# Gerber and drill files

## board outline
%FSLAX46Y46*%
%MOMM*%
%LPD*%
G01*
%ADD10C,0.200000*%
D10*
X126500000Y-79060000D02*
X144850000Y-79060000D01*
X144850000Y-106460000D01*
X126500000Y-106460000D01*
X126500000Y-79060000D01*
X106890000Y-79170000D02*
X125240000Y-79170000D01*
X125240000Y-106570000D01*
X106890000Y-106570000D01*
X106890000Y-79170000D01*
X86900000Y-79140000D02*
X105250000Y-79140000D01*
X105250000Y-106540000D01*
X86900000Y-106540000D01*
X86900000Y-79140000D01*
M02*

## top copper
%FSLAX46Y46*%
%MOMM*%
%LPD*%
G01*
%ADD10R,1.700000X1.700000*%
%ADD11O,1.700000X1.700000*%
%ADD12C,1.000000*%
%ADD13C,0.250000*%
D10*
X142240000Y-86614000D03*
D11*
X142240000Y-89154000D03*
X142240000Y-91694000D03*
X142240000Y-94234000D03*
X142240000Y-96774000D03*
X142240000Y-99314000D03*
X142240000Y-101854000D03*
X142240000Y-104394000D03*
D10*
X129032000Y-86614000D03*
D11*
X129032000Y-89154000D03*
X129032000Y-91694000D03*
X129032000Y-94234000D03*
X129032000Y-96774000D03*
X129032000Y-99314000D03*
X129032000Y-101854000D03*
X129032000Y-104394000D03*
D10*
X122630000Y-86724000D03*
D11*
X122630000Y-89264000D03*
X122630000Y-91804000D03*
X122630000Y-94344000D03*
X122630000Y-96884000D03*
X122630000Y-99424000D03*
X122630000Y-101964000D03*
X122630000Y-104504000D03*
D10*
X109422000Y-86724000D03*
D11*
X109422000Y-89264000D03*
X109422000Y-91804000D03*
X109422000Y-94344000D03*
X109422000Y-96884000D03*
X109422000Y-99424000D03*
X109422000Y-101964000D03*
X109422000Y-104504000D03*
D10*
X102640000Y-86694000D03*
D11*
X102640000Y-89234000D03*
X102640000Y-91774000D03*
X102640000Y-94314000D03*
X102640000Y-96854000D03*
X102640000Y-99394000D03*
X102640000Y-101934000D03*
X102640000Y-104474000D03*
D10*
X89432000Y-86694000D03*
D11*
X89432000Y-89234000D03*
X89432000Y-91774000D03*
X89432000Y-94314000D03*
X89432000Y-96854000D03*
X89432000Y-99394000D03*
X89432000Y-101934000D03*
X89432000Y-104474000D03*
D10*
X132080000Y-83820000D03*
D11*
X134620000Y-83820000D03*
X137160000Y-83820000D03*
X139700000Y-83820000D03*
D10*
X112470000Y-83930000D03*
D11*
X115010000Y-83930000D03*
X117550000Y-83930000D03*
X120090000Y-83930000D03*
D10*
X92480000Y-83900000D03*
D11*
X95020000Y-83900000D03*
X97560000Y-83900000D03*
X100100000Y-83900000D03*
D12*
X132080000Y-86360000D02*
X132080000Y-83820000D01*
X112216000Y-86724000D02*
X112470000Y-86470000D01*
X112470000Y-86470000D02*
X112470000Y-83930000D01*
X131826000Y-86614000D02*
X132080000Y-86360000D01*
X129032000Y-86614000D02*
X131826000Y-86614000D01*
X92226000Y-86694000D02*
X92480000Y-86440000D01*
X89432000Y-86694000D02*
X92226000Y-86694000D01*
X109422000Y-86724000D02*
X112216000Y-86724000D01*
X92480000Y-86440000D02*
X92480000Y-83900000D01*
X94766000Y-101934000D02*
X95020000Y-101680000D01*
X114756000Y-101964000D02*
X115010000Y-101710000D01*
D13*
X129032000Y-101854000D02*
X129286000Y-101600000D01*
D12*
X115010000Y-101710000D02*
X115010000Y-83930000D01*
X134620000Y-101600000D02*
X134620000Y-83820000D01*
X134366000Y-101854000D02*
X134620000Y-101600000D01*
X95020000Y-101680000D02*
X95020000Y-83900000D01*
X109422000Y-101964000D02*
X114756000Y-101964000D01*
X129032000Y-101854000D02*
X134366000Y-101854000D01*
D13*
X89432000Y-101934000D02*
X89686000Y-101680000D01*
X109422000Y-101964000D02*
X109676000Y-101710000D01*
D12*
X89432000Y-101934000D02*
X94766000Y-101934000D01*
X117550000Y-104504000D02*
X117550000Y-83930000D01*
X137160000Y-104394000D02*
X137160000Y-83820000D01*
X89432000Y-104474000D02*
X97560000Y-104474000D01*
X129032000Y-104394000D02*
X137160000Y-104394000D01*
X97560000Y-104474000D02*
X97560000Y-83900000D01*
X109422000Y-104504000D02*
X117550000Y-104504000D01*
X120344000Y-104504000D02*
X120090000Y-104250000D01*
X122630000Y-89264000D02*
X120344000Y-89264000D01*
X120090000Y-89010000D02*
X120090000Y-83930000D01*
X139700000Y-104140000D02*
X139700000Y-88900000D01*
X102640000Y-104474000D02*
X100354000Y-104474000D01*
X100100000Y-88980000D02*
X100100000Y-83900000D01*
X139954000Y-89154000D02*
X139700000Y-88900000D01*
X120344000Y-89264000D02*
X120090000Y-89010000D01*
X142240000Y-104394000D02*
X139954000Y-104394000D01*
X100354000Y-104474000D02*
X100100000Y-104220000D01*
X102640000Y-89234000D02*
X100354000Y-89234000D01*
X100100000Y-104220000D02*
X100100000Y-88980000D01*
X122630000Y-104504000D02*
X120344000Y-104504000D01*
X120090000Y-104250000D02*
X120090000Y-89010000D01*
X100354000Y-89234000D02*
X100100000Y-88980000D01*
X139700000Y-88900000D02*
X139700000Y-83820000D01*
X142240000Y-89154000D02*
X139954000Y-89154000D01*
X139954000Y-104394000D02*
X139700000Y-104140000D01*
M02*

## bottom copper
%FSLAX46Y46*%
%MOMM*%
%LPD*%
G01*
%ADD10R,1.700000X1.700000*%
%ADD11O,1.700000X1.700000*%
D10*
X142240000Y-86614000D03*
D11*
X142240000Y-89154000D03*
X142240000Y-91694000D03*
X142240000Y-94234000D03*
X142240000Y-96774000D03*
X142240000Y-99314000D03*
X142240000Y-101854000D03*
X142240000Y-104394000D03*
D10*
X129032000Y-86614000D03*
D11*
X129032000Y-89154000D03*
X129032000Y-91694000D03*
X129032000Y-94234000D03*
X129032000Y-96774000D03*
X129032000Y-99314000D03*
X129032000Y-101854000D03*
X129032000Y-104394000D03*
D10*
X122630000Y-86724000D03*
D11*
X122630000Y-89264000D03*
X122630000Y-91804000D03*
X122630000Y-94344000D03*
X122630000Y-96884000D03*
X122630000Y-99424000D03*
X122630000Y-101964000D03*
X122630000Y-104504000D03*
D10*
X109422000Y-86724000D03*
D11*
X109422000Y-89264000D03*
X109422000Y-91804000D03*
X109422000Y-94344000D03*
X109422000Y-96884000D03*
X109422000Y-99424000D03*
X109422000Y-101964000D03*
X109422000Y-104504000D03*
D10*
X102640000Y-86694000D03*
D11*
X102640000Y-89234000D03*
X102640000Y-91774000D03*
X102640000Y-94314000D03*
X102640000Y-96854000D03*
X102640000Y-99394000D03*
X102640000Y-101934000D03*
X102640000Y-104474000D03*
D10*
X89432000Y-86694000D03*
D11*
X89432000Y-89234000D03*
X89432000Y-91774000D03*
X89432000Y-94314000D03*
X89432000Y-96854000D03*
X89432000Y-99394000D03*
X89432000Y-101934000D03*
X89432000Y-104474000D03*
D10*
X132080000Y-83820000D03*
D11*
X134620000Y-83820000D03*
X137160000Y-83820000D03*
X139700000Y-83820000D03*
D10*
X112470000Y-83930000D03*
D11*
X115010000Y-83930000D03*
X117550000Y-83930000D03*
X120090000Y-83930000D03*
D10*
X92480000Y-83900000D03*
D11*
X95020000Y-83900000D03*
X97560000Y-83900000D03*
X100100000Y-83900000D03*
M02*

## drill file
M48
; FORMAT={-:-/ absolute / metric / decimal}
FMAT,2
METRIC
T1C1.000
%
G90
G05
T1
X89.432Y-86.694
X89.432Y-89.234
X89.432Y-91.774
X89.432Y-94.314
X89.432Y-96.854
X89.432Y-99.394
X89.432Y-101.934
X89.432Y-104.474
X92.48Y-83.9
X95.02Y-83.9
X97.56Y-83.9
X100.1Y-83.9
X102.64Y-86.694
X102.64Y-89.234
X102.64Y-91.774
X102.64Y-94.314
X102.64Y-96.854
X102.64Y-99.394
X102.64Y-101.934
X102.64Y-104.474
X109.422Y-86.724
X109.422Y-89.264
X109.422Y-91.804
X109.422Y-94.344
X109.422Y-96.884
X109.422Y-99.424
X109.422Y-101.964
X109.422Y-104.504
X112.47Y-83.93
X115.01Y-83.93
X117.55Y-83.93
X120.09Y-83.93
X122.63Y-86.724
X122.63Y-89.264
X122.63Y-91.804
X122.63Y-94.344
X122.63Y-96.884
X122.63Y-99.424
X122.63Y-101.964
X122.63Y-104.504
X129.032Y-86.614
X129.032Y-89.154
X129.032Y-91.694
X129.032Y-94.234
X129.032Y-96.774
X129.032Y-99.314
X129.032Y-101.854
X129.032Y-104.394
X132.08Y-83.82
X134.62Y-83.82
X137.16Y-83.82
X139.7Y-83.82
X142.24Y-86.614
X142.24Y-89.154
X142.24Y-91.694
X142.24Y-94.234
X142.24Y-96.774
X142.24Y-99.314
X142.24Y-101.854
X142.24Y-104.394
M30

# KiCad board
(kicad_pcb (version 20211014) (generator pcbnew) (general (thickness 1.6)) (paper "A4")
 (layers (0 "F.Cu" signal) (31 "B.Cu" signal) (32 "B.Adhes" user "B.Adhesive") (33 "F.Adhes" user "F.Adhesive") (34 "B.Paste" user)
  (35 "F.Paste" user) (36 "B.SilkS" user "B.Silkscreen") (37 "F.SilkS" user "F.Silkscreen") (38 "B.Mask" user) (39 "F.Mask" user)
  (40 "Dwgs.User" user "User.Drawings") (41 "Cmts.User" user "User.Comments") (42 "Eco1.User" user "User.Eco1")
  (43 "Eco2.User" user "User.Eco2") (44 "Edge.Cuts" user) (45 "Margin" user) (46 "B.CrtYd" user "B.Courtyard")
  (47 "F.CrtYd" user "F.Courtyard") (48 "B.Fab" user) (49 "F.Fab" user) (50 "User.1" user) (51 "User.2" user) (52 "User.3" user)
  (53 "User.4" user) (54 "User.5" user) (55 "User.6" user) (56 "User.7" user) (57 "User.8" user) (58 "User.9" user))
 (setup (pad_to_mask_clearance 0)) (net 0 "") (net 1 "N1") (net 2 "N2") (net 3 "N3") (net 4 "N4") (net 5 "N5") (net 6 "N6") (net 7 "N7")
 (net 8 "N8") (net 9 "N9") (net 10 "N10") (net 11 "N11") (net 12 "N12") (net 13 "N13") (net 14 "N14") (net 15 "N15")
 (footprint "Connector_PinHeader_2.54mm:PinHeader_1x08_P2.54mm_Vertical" (layer "F.Cu") (at 142.24 86.614)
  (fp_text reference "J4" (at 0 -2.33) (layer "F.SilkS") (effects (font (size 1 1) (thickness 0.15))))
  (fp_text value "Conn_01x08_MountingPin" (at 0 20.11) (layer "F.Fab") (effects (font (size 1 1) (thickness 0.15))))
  (pad "1" thru_hole rect (at 0 0) (size 1.7 1.7) (drill 1) (layers *.Cu *.Mask) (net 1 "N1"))
  (pad "2" thru_hole oval (at 0 2.54) (size 1.7 1.7) (drill 1) (layers *.Cu *.Mask) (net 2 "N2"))
  (pad "3" thru_hole oval (at 0 5.08) (size 1.7 1.7) (drill 1) (layers *.Cu *.Mask) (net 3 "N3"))
  (pad "4" thru_hole oval (at 0 7.62) (size 1.7 1.7) (drill 1) (layers *.Cu *.Mask) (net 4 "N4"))
  (pad "5" thru_hole oval (at 0 10.16) (size 1.7 1.7) (drill 1) (layers *.Cu *.Mask) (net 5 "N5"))
  (pad "6" thru_hole oval (at 0 12.7) (size 1.7 1.7) (drill 1) (layers *.Cu *.Mask) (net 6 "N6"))
  (pad "7" thru_hole oval (at 0 15.24) (size 1.7 1.7) (drill 1) (layers *.Cu *.Mask) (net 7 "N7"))
  (pad "8" thru_hole oval (at 0 17.78) (size 1.7 1.7) (drill 1) (layers *.Cu *.Mask) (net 2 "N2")))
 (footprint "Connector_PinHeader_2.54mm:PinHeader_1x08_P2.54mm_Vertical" (layer "F.Cu") (at 129.032 86.614)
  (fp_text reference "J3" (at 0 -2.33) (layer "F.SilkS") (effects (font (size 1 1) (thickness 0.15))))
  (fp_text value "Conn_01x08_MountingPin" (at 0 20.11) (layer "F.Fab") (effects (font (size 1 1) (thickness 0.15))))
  (pad "1" thru_hole rect (at 0 0) (size 1.7 1.7) (drill 1) (layers *.Cu *.Mask) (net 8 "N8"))
  (pad "2" thru_hole oval (at 0 2.54) (size 1.7 1.7) (drill 1) (layers *.Cu *.Mask) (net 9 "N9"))
  (pad "3" thru_hole oval (at 0 5.08) (size 1.7 1.7) (drill 1) (layers *.Cu *.Mask) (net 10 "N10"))
  (pad "4" thru_hole oval (at 0 7.62) (size 1.7 1.7) (drill 1) (layers *.Cu *.Mask) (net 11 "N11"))
  (pad "5" thru_hole oval (at 0 10.16) (size 1.7 1.7) (drill 1) (layers *.Cu *.Mask) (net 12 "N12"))
  (pad "6" thru_hole oval (at 0 12.7) (size 1.7 1.7) (drill 1) (layers *.Cu *.Mask) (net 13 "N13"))
  (pad "7" thru_hole oval (at 0 15.24) (size 1.7 1.7) (drill 1) (layers *.Cu *.Mask) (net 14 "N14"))
  (pad "8" thru_hole oval (at 0 17.78) (size 1.7 1.7) (drill 1) (layers *.Cu *.Mask) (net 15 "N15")))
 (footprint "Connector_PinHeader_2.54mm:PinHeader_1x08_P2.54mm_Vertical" (layer "F.Cu") (at 122.63 86.724)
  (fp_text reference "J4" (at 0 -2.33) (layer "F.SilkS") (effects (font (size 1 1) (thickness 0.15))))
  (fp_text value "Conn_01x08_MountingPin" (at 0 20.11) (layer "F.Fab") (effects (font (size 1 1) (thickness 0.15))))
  (pad "1" thru_hole rect (at 0 0) (size 1.7 1.7) (drill 1) (layers *.Cu *.Mask) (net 1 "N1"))
  (pad "2" thru_hole oval (at 0 2.54) (size 1.7 1.7) (drill 1) (layers *.Cu *.Mask) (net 2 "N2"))
  (pad "3" thru_hole oval (at 0 5.08) (size 1.7 1.7) (drill 1) (layers *.Cu *.Mask) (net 3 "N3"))
  (pad "4" thru_hole oval (at 0 7.62) (size 1.7 1.7) (drill 1) (layers *.Cu *.Mask) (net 4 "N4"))
  (pad "5" thru_hole oval (at 0 10.16) (size 1.7 1.7) (drill 1) (layers *.Cu *.Mask) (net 5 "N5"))
  (pad "6" thru_hole oval (at 0 12.7) (size 1.7 1.7) (drill 1) (layers *.Cu *.Mask) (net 6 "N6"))
  (pad "7" thru_hole oval (at 0 15.24) (size 1.7 1.7) (drill 1) (layers *.Cu *.Mask) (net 7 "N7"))
  (pad "8" thru_hole oval (at 0 17.78) (size 1.7 1.7) (drill 1) (layers *.Cu *.Mask) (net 2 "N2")))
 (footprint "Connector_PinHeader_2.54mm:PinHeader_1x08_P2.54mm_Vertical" (layer "F.Cu") (at 109.422 86.724)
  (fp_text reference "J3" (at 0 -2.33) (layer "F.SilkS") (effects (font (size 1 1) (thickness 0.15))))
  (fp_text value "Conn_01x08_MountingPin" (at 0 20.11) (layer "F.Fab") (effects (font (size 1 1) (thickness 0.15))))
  (pad "1" thru_hole rect (at 0 0) (size 1.7 1.7) (drill 1) (layers *.Cu *.Mask) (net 8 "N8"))
  (pad "2" thru_hole oval (at 0 2.54) (size 1.7 1.7) (drill 1) (layers *.Cu *.Mask) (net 9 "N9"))
  (pad "3" thru_hole oval (at 0 5.08) (size 1.7 1.7) (drill 1) (layers *.Cu *.Mask) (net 10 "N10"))
  (pad "4" thru_hole oval (at 0 7.62) (size 1.7 1.7) (drill 1) (layers *.Cu *.Mask) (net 11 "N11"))
  (pad "5" thru_hole oval (at 0 10.16) (size 1.7 1.7) (drill 1) (layers *.Cu *.Mask) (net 12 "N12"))
  (pad "6" thru_hole oval (at 0 12.7) (size 1.7 1.7) (drill 1) (layers *.Cu *.Mask) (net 13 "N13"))
  (pad "7" thru_hole oval (at 0 15.24) (size 1.7 1.7) (drill 1) (layers *.Cu *.Mask) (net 14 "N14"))
  (pad "8" thru_hole oval (at 0 17.78) (size 1.7 1.7) (drill 1) (layers *.Cu *.Mask) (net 15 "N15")))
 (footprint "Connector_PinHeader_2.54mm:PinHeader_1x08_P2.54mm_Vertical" (layer "F.Cu") (at 102.64 86.694)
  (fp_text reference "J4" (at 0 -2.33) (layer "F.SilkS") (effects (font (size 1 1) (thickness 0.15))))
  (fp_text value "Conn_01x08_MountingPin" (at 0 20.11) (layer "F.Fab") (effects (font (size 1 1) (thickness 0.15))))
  (pad "1" thru_hole rect (at 0 0) (size 1.7 1.7) (drill 1) (layers *.Cu *.Mask) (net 1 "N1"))
  (pad "2" thru_hole oval (at 0 2.54) (size 1.7 1.7) (drill 1) (layers *.Cu *.Mask) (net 2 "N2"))
  (pad "3" thru_hole oval (at 0 5.08) (size 1.7 1.7) (drill 1) (layers *.Cu *.Mask) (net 3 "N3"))
  (pad "4" thru_hole oval (at 0 7.62) (size 1.7 1.7) (drill 1) (layers *.Cu *.Mask) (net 4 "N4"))
  (pad "5" thru_hole oval (at 0 10.16) (size 1.7 1.7) (drill 1) (layers *.Cu *.Mask) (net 5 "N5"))
  (pad "6" thru_hole oval (at 0 12.7) (size 1.7 1.7) (drill 1) (layers *.Cu *.Mask) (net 6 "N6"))
  (pad "7" thru_hole oval (at 0 15.24) (size 1.7 1.7) (drill 1) (layers *.Cu *.Mask) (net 7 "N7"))
  (pad "8" thru_hole oval (at 0 17.78) (size 1.7 1.7) (drill 1) (layers *.Cu *.Mask) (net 2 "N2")))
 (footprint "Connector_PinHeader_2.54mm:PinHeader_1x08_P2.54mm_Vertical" (layer "F.Cu") (at 89.432 86.694)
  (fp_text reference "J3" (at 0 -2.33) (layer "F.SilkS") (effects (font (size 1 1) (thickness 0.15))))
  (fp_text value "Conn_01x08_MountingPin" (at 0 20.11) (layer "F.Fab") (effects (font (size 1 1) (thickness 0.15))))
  (pad "1" thru_hole rect (at 0 0) (size 1.7 1.7) (drill 1) (layers *.Cu *.Mask) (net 8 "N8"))
  (pad "2" thru_hole oval (at 0 2.54) (size 1.7 1.7) (drill 1) (layers *.Cu *.Mask) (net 9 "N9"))
  (pad "3" thru_hole oval (at 0 5.08) (size 1.7 1.7) (drill 1) (layers *.Cu *.Mask) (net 10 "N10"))
  (pad "4" thru_hole oval (at 0 7.62) (size 1.7 1.7) (drill 1) (layers *.Cu *.Mask) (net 11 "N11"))
  (pad "5" thru_hole oval (at 0 10.16) (size 1.7 1.7) (drill 1) (layers *.Cu *.Mask) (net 12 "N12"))
  (pad "6" thru_hole oval (at 0 12.7) (size 1.7 1.7) (drill 1) (layers *.Cu *.Mask) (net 13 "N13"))
  (pad "7" thru_hole oval (at 0 15.24) (size 1.7 1.7) (drill 1) (layers *.Cu *.Mask) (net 14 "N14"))
  (pad "8" thru_hole oval (at 0 17.78) (size 1.7 1.7) (drill 1) (layers *.Cu *.Mask) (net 15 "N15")))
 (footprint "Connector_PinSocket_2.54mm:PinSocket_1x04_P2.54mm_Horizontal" (layer "B.Cu") (at 132.08 83.82 -90)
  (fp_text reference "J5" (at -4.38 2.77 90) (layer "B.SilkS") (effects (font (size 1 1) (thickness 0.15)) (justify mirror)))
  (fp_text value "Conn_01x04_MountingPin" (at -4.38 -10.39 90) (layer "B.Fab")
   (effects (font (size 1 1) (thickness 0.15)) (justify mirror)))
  (pad "1" thru_hole rect (at 0 0 270) (size 1.7 1.7) (drill 1) (layers *.Cu *.Mask) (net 8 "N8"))
  (pad "2" thru_hole oval (at 0 -2.54 270) (size 1.7 1.7) (drill 1) (layers *.Cu *.Mask) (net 14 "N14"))
  (pad "3" thru_hole oval (at 0 -5.08 270) (size 1.7 1.7) (drill 1) (layers *.Cu *.Mask) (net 15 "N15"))
  (pad "4" thru_hole oval (at 0 -7.62 270) (size 1.7 1.7) (drill 1) (layers *.Cu *.Mask) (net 2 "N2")))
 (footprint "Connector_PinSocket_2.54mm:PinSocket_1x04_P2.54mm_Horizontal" (layer "B.Cu") (at 112.47 83.93 -90)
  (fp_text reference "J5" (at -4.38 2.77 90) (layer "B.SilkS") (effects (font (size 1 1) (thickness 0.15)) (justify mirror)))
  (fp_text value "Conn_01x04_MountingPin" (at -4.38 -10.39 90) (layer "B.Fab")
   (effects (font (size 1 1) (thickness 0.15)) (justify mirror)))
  (pad "1" thru_hole rect (at 0 0 270) (size 1.7 1.7) (drill 1) (layers *.Cu *.Mask) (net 8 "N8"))
  (pad "2" thru_hole oval (at 0 -2.54 270) (size 1.7 1.7) (drill 1) (layers *.Cu *.Mask) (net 14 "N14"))
  (pad "3" thru_hole oval (at 0 -5.08 270) (size 1.7 1.7) (drill 1) (layers *.Cu *.Mask) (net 15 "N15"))
  (pad "4" thru_hole oval (at 0 -7.62 270) (size 1.7 1.7) (drill 1) (layers *.Cu *.Mask) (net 2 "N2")))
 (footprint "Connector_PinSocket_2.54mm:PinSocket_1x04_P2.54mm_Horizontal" (layer "B.Cu") (at 92.48 83.9 -90)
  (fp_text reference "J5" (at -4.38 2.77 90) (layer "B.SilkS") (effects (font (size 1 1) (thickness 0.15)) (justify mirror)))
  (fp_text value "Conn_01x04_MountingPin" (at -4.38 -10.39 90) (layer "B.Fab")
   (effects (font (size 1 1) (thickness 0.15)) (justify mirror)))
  (pad "1" thru_hole rect (at 0 0 270) (size 1.7 1.7) (drill 1) (layers *.Cu *.Mask) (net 8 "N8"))
  (pad "2" thru_hole oval (at 0 -2.54 270) (size 1.7 1.7) (drill 1) (layers *.Cu *.Mask) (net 14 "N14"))
  (pad "3" thru_hole oval (at 0 -5.08 270) (size 1.7 1.7) (drill 1) (layers *.Cu *.Mask) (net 15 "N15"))
  (pad "4" thru_hole oval (at 0 -7.62 270) (size 1.7 1.7) (drill 1) (layers *.Cu *.Mask) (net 2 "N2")))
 (gr_rect (start 126.5 79.06) (end 144.85 106.46) (layer "Edge.Cuts") (width 0.2) (fill none))
 (gr_rect (start 106.89 79.17) (end 125.24 106.57) (layer "Edge.Cuts") (width 0.2) (fill none))
 (gr_rect (start 86.9 79.14) (end 105.25 106.54) (layer "Edge.Cuts") (width 0.2) (fill none))
 (segment (start 132.08 86.36) (end 132.08 83.82) (width 1) (layer "F.Cu") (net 8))
 (segment (start 112.216 86.724) (end 112.47 86.47) (width 1) (layer "F.Cu") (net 8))
 (segment (start 112.47 86.47) (end 112.47 83.93) (width 1) (layer "F.Cu") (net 8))
 (segment (start 131.826 86.614) (end 132.08 86.36) (width 1) (layer "F.Cu") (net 8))
 (segment (start 129.032 86.614) (end 131.826 86.614) (width 1) (layer "F.Cu") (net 8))
 (segment (start 92.226 86.694) (end 92.48 86.44) (width 1) (layer "F.Cu") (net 8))
 (segment (start 89.432 86.694) (end 92.226 86.694) (width 1) (layer "F.Cu") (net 8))
 (segment (start 109.422 86.724) (end 112.216 86.724) (width 1) (layer "F.Cu") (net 8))
 (segment (start 92.48 86.44) (end 92.48 83.9) (width 1) (layer "F.Cu") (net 8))
 (segment (start 94.766 101.934) (end 95.02 101.68) (width 1) (layer "F.Cu") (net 14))
 (segment (start 114.756 101.964) (end 115.01 101.71) (width 1) (layer "F.Cu") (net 14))
 (segment (start 129.032 101.854) (end 129.286 101.6) (width 0.25) (layer "F.Cu") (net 14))
 (segment (start 115.01 101.71) (end 115.01 83.93) (width 1) (layer "F.Cu") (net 14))
 (segment (start 134.62 101.6) (end 134.62 83.82) (width 1) (layer "F.Cu") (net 14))
 (segment (start 134.366 101.854) (end 134.62 101.6) (width 1) (layer "F.Cu") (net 14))
 (segment (start 95.02 101.68) (end 95.02 83.9) (width 1) (layer "F.Cu") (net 14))
 (segment (start 109.422 101.964) (end 114.756 101.964) (width 1) (layer "F.Cu") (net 14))
 (segment (start 129.032 101.854) (end 134.366 101.854) (width 1) (layer "F.Cu") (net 14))
 (segment (start 89.432 101.934) (end 89.686 101.68) (width 0.25) (layer "F.Cu") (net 14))
 (segment (start 109.422 101.964) (end 109.676 101.71) (width 0.25) (layer "F.Cu") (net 14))
 (segment (start 89.432 101.934) (end 94.766 101.934) (width 1) (layer "F.Cu") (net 14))
 (segment (start 117.55 104.504) (end 117.55 83.93) (width 1) (layer "F.Cu") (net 15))
 (segment (start 137.16 104.394) (end 137.16 83.82) (width 1) (layer "F.Cu") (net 15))
 (segment (start 89.432 104.474) (end 97.56 104.474) (width 1) (layer "F.Cu") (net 15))
 (segment (start 129.032 104.394) (end 137.16 104.394) (width 1) (layer "F.Cu") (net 15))
 (segment (start 97.56 104.474) (end 97.56 83.9) (width 1) (layer "F.Cu") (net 15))
 (segment (start 109.422 104.504) (end 117.55 104.504) (width 1) (layer "F.Cu") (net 15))
 (segment (start 120.344 104.504) (end 120.09 104.25) (width 1) (layer "F.Cu") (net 2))
 (segment (start 122.63 89.264) (end 120.344 89.264) (width 1) (layer "F.Cu") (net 2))
 (segment (start 120.09 89.01) (end 120.09 83.93) (width 1) (layer "F.Cu") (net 2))
 (segment (start 139.7 104.14) (end 139.7 88.9) (width 1) (layer "F.Cu") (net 2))
 (segment (start 102.64 104.474) (end 100.354 104.474) (width 1) (layer "F.Cu") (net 2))
 (segment (start 100.1 88.98) (end 100.1 83.9) (width 1) (layer "F.Cu") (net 2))
 (segment (start 139.954 89.154) (end 139.7 88.9) (width 1) (layer "F.Cu") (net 2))
 (segment (start 120.344 89.264) (end 120.09 89.01) (width 1) (layer "F.Cu") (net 2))
 (segment (start 142.24 104.394) (end 139.954 104.394) (width 1) (layer "F.Cu") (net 2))
 (segment (start 100.354 104.474) (end 100.1 104.22) (width 1) (layer "F.Cu") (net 2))
 (segment (start 102.64 89.234) (end 100.354 89.234) (width 1) (layer "F.Cu") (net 2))
 (segment (start 100.1 104.22) (end 100.1 88.98) (width 1) (layer "F.Cu") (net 2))
 (segment (start 122.63 104.504) (end 120.344 104.504) (width 1) (layer "F.Cu") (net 2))
 (segment (start 120.09 104.25) (end 120.09 89.01) (width 1) (layer "F.Cu") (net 2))
 (segment (start 100.354 89.234) (end 100.1 88.98) (width 1) (layer "F.Cu") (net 2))
 (segment (start 139.7 88.9) (end 139.7 83.82) (width 1) (layer "F.Cu") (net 2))
 (segment (start 142.24 89.154) (end 139.954 89.154) (width 1) (layer "F.Cu") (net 2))
 (segment (start 139.954 104.394) (end 139.7 104.14) (width 1) (layer "F.Cu") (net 2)))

